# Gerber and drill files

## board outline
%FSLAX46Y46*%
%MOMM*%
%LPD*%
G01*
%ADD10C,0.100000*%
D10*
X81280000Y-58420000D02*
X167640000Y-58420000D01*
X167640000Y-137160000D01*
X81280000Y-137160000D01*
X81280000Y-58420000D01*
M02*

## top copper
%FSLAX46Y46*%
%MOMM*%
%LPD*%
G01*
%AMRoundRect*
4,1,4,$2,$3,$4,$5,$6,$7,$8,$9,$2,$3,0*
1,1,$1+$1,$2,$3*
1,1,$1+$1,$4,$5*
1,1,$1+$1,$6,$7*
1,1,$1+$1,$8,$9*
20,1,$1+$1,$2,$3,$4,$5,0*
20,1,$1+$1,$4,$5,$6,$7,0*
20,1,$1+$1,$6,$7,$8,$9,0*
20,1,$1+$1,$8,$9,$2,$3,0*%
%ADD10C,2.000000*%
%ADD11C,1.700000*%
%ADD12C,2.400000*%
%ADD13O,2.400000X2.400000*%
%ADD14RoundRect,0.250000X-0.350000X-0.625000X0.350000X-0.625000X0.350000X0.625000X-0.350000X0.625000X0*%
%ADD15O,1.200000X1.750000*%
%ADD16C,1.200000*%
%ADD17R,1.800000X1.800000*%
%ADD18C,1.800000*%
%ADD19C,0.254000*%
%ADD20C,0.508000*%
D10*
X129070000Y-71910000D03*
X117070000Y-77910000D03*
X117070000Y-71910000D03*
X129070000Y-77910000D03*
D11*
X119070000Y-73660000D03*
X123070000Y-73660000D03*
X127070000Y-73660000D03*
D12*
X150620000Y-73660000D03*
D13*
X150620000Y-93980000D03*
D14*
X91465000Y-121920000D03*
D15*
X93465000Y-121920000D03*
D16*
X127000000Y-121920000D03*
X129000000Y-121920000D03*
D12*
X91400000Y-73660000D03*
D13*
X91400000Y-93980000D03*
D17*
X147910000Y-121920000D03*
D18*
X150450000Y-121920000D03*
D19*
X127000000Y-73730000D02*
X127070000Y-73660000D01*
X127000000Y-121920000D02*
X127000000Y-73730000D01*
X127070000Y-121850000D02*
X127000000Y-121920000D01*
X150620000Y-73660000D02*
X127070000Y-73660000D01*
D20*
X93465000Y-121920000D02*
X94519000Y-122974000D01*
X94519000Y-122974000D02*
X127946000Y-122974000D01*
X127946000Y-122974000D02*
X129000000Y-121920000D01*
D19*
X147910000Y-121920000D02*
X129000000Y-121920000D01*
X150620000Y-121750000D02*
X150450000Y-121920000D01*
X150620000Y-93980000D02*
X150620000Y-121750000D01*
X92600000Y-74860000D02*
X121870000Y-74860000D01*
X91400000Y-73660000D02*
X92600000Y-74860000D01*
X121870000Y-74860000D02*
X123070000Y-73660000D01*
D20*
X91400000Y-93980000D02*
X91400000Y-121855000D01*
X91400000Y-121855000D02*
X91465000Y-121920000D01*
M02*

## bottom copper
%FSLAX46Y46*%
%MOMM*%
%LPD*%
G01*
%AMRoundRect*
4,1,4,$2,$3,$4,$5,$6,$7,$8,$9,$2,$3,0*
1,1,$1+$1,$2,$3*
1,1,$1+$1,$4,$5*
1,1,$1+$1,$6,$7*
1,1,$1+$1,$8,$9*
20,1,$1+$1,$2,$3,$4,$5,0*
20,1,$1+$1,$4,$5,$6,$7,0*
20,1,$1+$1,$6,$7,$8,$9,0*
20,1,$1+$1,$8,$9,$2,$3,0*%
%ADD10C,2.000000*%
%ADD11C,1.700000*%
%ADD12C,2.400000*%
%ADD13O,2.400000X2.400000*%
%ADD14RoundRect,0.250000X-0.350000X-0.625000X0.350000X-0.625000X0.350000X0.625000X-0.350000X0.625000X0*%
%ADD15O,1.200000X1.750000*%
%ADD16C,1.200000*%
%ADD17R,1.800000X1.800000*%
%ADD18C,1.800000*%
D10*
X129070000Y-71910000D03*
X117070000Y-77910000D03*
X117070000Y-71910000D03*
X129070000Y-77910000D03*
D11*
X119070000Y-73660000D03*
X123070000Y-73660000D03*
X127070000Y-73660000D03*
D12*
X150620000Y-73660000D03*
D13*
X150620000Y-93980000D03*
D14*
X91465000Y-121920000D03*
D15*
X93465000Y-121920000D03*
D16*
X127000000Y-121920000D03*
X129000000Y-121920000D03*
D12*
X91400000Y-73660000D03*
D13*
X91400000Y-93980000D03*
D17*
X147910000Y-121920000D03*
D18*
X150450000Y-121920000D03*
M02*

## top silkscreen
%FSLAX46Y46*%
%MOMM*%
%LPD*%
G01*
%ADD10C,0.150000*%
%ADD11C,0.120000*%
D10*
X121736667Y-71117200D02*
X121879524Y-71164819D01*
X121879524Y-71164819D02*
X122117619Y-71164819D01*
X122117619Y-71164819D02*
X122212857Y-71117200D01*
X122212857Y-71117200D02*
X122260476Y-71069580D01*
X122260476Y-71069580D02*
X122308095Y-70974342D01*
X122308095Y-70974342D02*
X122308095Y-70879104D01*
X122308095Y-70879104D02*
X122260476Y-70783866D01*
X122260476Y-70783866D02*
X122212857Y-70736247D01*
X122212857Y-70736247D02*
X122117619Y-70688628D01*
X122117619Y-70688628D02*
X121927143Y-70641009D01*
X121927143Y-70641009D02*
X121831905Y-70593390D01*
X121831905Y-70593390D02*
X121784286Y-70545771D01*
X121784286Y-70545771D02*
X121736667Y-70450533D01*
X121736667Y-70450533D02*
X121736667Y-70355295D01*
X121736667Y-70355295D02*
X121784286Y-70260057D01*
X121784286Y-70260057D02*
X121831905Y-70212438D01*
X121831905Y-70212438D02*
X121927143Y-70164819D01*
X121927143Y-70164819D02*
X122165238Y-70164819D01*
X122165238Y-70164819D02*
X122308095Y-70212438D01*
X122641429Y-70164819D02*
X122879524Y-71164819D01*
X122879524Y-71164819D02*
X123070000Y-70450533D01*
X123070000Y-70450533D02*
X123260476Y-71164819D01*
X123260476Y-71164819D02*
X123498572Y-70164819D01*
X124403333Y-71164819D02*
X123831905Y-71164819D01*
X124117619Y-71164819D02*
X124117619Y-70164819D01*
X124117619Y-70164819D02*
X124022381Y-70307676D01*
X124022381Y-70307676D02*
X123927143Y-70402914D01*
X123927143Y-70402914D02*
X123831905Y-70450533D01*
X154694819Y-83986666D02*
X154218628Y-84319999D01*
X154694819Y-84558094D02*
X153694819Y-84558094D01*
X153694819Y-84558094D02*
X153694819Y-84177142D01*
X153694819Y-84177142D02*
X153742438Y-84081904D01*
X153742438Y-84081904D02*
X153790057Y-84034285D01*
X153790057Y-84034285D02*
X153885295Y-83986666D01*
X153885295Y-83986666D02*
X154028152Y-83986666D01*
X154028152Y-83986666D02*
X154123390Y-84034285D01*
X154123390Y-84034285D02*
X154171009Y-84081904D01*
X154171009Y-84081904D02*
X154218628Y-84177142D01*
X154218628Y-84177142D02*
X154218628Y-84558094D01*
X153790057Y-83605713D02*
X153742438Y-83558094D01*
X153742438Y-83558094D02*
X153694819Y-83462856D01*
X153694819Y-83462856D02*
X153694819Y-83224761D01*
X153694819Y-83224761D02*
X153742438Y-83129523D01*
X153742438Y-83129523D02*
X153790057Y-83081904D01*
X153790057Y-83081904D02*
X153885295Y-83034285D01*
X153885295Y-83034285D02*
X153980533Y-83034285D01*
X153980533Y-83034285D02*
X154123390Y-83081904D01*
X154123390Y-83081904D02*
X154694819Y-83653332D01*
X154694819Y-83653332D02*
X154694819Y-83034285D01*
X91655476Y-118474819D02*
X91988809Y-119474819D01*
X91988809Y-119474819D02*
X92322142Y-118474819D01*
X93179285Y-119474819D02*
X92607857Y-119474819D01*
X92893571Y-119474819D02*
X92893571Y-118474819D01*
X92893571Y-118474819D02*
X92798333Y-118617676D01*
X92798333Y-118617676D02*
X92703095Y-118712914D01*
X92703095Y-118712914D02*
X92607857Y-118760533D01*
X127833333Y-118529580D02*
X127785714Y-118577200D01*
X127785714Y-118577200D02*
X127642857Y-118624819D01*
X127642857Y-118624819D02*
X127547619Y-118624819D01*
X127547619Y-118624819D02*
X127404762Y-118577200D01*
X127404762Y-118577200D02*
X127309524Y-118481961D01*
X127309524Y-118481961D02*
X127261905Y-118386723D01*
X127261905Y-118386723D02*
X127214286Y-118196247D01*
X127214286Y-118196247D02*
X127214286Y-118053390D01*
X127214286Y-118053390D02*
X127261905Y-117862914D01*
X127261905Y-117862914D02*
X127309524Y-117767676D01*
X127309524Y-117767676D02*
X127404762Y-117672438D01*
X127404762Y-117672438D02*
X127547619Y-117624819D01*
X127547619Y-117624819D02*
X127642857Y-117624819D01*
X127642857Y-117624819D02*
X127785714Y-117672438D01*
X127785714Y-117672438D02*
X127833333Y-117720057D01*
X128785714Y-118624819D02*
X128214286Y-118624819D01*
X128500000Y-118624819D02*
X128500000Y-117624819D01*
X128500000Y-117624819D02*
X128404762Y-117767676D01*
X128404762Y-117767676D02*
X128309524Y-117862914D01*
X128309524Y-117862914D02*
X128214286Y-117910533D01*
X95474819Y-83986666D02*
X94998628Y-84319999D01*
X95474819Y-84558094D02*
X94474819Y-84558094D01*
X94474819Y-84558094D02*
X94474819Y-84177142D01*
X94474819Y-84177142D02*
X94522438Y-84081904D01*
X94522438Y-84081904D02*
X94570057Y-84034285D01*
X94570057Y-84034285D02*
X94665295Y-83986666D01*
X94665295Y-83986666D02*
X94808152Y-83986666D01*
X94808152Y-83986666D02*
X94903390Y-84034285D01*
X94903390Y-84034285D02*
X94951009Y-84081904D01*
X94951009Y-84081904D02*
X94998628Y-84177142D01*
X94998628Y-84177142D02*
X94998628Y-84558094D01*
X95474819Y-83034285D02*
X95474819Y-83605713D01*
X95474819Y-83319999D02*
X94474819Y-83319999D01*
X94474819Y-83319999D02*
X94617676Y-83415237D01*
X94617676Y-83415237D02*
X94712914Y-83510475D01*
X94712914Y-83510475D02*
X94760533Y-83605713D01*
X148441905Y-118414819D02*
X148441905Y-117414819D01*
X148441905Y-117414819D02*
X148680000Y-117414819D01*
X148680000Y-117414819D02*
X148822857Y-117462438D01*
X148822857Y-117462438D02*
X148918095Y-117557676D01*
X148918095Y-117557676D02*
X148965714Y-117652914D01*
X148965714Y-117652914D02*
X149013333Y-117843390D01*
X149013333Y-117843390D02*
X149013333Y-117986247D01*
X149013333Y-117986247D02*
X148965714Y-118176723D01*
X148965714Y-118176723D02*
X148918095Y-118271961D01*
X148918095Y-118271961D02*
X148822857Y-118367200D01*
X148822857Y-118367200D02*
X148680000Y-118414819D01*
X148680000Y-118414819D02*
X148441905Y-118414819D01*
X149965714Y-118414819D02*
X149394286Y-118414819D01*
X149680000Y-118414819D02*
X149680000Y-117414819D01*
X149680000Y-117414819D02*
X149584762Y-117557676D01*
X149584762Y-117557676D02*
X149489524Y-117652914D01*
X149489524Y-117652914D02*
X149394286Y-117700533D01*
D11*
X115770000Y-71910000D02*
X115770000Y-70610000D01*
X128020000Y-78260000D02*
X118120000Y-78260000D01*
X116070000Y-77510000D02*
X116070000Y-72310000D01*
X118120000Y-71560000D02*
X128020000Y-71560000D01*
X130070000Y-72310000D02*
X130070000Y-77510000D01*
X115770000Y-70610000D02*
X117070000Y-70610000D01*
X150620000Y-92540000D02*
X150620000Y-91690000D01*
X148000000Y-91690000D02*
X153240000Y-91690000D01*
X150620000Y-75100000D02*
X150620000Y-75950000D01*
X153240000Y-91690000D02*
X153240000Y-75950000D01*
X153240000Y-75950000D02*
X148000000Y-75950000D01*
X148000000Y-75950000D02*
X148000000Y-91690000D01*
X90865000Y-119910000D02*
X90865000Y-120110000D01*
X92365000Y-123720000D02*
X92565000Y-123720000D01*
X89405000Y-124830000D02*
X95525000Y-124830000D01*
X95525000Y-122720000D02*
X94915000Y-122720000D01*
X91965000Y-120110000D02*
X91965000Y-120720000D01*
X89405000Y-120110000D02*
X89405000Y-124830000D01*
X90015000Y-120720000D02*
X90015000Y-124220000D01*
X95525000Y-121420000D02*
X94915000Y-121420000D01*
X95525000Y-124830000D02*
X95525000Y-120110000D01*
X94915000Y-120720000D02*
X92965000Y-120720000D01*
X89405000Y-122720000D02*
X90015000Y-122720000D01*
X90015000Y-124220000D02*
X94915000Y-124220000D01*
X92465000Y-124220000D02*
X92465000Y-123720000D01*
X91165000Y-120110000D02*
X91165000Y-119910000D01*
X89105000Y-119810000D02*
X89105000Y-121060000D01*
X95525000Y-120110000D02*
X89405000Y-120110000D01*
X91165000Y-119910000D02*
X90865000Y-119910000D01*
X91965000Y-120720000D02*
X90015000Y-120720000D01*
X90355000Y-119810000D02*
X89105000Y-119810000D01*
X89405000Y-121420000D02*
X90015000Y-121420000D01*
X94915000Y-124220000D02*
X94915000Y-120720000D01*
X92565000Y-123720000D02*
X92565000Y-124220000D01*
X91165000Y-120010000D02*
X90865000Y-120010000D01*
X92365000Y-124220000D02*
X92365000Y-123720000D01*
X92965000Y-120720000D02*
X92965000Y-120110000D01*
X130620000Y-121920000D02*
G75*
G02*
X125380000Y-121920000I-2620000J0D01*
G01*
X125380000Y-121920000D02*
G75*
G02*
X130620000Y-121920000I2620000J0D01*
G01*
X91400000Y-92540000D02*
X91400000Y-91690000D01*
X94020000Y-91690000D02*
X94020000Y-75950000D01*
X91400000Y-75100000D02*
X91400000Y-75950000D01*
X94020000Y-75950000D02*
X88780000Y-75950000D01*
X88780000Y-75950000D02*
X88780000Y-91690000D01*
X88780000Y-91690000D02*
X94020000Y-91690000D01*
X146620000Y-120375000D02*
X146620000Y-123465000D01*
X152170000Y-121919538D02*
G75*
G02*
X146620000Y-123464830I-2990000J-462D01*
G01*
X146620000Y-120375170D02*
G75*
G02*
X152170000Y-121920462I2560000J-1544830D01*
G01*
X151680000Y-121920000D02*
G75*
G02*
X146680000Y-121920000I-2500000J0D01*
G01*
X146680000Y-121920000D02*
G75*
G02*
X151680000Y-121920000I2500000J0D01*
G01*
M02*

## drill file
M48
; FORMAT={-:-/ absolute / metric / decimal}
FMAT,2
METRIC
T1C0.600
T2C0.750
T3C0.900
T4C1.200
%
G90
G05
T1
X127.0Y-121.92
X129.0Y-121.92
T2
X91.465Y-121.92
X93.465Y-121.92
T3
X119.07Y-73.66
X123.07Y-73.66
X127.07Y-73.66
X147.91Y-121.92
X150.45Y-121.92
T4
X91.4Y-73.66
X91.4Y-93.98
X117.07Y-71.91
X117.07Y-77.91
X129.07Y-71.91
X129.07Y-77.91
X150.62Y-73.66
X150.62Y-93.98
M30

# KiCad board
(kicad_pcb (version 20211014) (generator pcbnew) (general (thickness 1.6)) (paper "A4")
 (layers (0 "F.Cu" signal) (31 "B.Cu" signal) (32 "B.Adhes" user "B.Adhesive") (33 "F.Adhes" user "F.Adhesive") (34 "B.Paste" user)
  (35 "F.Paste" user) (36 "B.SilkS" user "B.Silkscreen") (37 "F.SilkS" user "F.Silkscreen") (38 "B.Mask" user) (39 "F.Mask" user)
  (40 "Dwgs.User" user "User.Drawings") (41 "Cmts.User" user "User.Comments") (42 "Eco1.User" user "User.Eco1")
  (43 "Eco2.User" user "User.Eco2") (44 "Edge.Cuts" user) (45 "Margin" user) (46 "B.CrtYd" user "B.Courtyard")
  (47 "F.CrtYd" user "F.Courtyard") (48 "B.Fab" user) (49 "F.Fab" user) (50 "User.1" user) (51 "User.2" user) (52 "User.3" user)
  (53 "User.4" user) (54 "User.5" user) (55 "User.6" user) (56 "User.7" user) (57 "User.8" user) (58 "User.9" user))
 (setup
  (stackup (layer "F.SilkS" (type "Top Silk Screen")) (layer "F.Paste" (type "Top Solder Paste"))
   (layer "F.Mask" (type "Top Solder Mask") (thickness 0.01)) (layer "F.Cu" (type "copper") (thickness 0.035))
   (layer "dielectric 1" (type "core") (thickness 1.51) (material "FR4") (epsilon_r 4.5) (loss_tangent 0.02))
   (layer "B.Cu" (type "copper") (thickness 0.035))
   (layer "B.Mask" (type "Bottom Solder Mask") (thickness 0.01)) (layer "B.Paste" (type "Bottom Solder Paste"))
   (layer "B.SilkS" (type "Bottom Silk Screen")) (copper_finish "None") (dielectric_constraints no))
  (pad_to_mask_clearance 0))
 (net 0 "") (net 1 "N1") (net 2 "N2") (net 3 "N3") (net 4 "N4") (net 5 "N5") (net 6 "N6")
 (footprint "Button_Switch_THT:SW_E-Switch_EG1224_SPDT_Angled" (layer "F.Cu") (at 119.07 73.66)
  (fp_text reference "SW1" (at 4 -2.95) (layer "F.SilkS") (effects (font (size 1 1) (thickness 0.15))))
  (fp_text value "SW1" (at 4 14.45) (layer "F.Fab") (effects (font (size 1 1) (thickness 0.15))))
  (fp_line (start -3.3 -1.75) (end -3.3 -3.05) (layer "F.SilkS") (width 0.12))
  (fp_line (start 8.95 4.6) (end -0.95 4.6) (layer "F.SilkS") (width 0.12))
  (fp_line (start -3 3.85) (end -3 -1.35) (layer "F.SilkS") (width 0.12))
  (fp_line (start -0.95 -2.1) (end 8.95 -2.1) (layer "F.SilkS") (width 0.12))
  (fp_line (start 11 -1.35) (end 11 3.85) (layer "F.SilkS") (width 0.12))
  (fp_line (start -3.3 -3.05) (end -2 -3.05) (layer "F.SilkS") (width 0.12))
  (pad "" thru_hole circle (at 10 -1.75) (size 2 2) (drill 1.2) (layers *.Cu *.Mask))
  (pad "" thru_hole circle (at -2 4.25) (size 2 2) (drill 1.2) (layers *.Cu *.Mask))
  (pad "" thru_hole circle (at -2 -1.75) (size 2 2) (drill 1.2) (layers *.Cu *.Mask))
  (pad "" thru_hole circle (at 10 4.25) (size 2 2) (drill 1.2) (layers *.Cu *.Mask))
  (pad "1" thru_hole circle (at 0 0) (size 1.7 1.7) (drill 0.9) (layers *.Cu *.Mask) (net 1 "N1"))
  (pad "2" thru_hole circle (at 4 0) (size 1.7 1.7) (drill 0.9) (layers *.Cu *.Mask) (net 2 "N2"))
  (pad "3" thru_hole circle (at 8 0) (size 1.7 1.7) (drill 0.9) (layers *.Cu *.Mask) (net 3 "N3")))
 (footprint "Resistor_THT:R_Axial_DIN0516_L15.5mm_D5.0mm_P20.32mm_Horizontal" (layer "F.Cu") (at 150.62 73.66 -90)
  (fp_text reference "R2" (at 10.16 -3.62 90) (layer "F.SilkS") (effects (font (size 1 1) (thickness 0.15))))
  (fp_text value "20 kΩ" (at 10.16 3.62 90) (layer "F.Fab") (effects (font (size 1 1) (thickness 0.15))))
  (fp_line (start 18.88 0) (end 18.03 0) (layer "F.SilkS") (width 0.12))
  (fp_line (start 18.03 2.62) (end 18.03 -2.62) (layer "F.SilkS") (width 0.12))
  (fp_line (start 1.44 0) (end 2.29 0) (layer "F.SilkS") (width 0.12))
  (fp_line (start 18.03 -2.62) (end 2.29 -2.62) (layer "F.SilkS") (width 0.12))
  (fp_line (start 2.29 -2.62) (end 2.29 2.62) (layer "F.SilkS") (width 0.12))
  (fp_line (start 2.29 2.62) (end 18.03 2.62) (layer "F.SilkS") (width 0.12))
  (pad "1" thru_hole circle (at 0 0 270) (size 2.4 2.4) (drill 1.2) (layers *.Cu *.Mask) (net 3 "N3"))
  (pad "2" thru_hole oval (at 20.32 0 270) (size 2.4 2.4) (drill 1.2) (layers *.Cu *.Mask) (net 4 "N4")))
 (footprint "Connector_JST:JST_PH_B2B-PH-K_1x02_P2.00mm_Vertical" (layer "F.Cu") (at 91.465 121.92)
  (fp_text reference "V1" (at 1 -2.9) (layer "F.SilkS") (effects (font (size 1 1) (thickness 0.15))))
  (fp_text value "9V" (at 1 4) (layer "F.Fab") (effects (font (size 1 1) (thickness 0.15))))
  (fp_line (start -0.6 -2.01) (end -0.6 -1.81) (layer "F.SilkS") (width 0.12))
  (fp_line (start 0.9 1.8) (end 1.1 1.8) (layer "F.SilkS") (width 0.12))
  (fp_line (start -2.06 2.91) (end 4.06 2.91) (layer "F.SilkS") (width 0.12))
  (fp_line (start 4.06 0.8) (end 3.45 0.8) (layer "F.SilkS") (width 0.12))
  (fp_line (start 0.5 -1.81) (end 0.5 -1.2) (layer "F.SilkS") (width 0.12))
  (fp_line (start -2.06 -1.81) (end -2.06 2.91) (layer "F.SilkS") (width 0.12))
  (fp_line (start -1.45 -1.2) (end -1.45 2.3) (layer "F.SilkS") (width 0.12))
  (fp_line (start 4.06 -0.5) (end 3.45 -0.5) (layer "F.SilkS") (width 0.12))
  (fp_line (start 4.06 2.91) (end 4.06 -1.81) (layer "F.SilkS") (width 0.12))
  (fp_line (start 3.45 -1.2) (end 1.5 -1.2) (layer "F.SilkS") (width 0.12))
  (fp_line (start -2.06 0.8) (end -1.45 0.8) (layer "F.SilkS") (width 0.12))
  (fp_line (start -1.45 2.3) (end 3.45 2.3) (layer "F.SilkS") (width 0.12))
  (fp_line (start 1 2.3) (end 1 1.8) (layer "F.SilkS") (width 0.12))
  (fp_line (start -0.3 -1.81) (end -0.3 -2.01) (layer "F.SilkS") (width 0.12))
  (fp_line (start -2.36 -2.11) (end -2.36 -0.86) (layer "F.SilkS") (width 0.12))
  (fp_line (start 4.06 -1.81) (end -2.06 -1.81) (layer "F.SilkS") (width 0.12))
  (fp_line (start -0.3 -2.01) (end -0.6 -2.01) (layer "F.SilkS") (width 0.12))
  (fp_line (start 0.5 -1.2) (end -1.45 -1.2) (layer "F.SilkS") (width 0.12))
  (fp_line (start -1.11 -2.11) (end -2.36 -2.11) (layer "F.SilkS") (width 0.12))
  (fp_line (start -2.06 -0.5) (end -1.45 -0.5) (layer "F.SilkS") (width 0.12))
  (fp_line (start 3.45 2.3) (end 3.45 -1.2) (layer "F.SilkS") (width 0.12))
  (fp_line (start 1.1 1.8) (end 1.1 2.3) (layer "F.SilkS") (width 0.12))
  (fp_line (start -0.3 -1.91) (end -0.6 -1.91) (layer "F.SilkS") (width 0.12))
  (fp_line (start 0.9 2.3) (end 0.9 1.8) (layer "F.SilkS") (width 0.12))
  (fp_line (start 1.5 -1.2) (end 1.5 -1.81) (layer "F.SilkS") (width 0.12))
  (pad "1" thru_hole roundrect (at 0 0) (size 1.2 1.75) (drill 0.75) (layers *.Cu *.Mask) (roundrect_rratio 0.208333) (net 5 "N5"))
  (pad "2" thru_hole oval (at 2 0) (size 1.2 1.75) (drill 0.75) (layers *.Cu *.Mask) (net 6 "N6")))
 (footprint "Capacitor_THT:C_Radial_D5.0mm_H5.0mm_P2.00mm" (layer "F.Cu") (at 127 121.92)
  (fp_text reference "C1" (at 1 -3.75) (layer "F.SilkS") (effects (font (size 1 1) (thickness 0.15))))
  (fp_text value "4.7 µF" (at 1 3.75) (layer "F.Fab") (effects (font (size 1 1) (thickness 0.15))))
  (fp_circle (center 1 0) (end 3.62 0) (layer "F.SilkS") (width 0.12) (fill none))
  (pad "1" thru_hole circle (at 0 0) (size 1.2 1.2) (drill 0.6) (layers *.Cu *.Mask) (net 3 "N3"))
  (pad "2" thru_hole circle (at 2 0) (size 1.2 1.2) (drill 0.6) (layers *.Cu *.Mask) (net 6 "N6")))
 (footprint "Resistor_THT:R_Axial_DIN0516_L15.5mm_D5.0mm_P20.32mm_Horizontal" (layer "F.Cu") (at 91.4 73.66 -90)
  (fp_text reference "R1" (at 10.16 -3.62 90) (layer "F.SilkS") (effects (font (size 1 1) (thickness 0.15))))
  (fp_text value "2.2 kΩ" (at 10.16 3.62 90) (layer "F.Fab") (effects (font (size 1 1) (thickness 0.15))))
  (fp_line (start 18.88 0) (end 18.03 0) (layer "F.SilkS") (width 0.12))
  (fp_line (start 18.03 -2.62) (end 2.29 -2.62) (layer "F.SilkS") (width 0.12))
  (fp_line (start 1.44 0) (end 2.29 0) (layer "F.SilkS") (width 0.12))
  (fp_line (start 2.29 -2.62) (end 2.29 2.62) (layer "F.SilkS") (width 0.12))
  (fp_line (start 2.29 2.62) (end 18.03 2.62) (layer "F.SilkS") (width 0.12))
  (fp_line (start 18.03 2.62) (end 18.03 -2.62) (layer "F.SilkS") (width 0.12))
  (pad "1" thru_hole circle (at 0 0 270) (size 2.4 2.4) (drill 1.2) (layers *.Cu *.Mask) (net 2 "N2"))
  (pad "2" thru_hole oval (at 20.32 0 270) (size 2.4 2.4) (drill 1.2) (layers *.Cu *.Mask) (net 5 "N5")))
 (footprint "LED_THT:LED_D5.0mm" (layer "F.Cu") (at 147.91 121.92)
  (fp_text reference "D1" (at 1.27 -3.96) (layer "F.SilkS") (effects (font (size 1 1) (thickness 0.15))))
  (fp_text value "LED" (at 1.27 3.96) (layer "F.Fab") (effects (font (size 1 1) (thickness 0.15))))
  (fp_line (start -1.29 -1.545) (end -1.29 1.545) (layer "F.SilkS") (width 0.12))
  (fp_arc (start 4.26 -0.000462) (mid 2.072002 2.880433) (end -1.29 1.54483) (layer "F.SilkS") (width 0.12))
  (fp_arc (start -1.29 -1.54483) (mid 2.072002 -2.880433) (end 4.26 0.000462) (layer "F.SilkS") (width 0.12))
  (fp_circle (center 1.27 0) (end 3.77 0) (layer "F.SilkS") (width 0.12) (fill none))
  (pad "1" thru_hole rect (at 0 0) (size 1.8 1.8) (drill 0.9) (layers *.Cu *.Mask) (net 6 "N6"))
  (pad "2" thru_hole circle (at 2.54 0) (size 1.8 1.8) (drill 0.9) (layers *.Cu *.Mask) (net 4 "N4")))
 (gr_rect (start 81.28 58.42) (end 167.64 137.16) (layer "Edge.Cuts") (width 0.1) (fill none))
 (segment (start 127 73.73) (end 127.07 73.66) (width 0.254) (layer "F.Cu") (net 3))
 (segment (start 127 121.92) (end 127 73.73) (width 0.254) (layer "F.Cu") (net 3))
 (segment (start 127.07 121.85) (end 127 121.92) (width 0.254) (layer "F.Cu") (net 3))
 (segment (start 150.62 73.66) (end 127.07 73.66) (width 0.254) (layer "F.Cu") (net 3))
 (segment (start 93.465 121.92) (end 94.519 122.974) (width 0.508) (layer "F.Cu") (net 6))
 (segment (start 94.519 122.974) (end 127.946 122.974) (width 0.508) (layer "F.Cu") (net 6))
 (segment (start 127.946 122.974) (end 129 121.92) (width 0.508) (layer "F.Cu") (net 6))
 (segment (start 147.91 121.92) (end 129 121.92) (width 0.254) (layer "F.Cu") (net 6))
 (segment (start 150.62 121.75) (end 150.45 121.92) (width 0.254) (layer "F.Cu") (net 4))
 (segment (start 150.62 93.98) (end 150.62 121.75) (width 0.254) (layer "F.Cu") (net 4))
 (segment (start 92.6 74.86) (end 121.87 74.86) (width 0.254) (layer "F.Cu") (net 2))
 (segment (start 91.4 73.66) (end 92.6 74.86) (width 0.254) (layer "F.Cu") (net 2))
 (segment (start 121.87 74.86) (end 123.07 73.66) (width 0.254) (layer "F.Cu") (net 2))
 (segment (start 91.4 93.98) (end 91.4 121.855) (width 0.508) (layer "F.Cu") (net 5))
 (segment (start 91.4 121.855) (end 91.465 121.92) (width 0.508) (layer "F.Cu") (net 5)))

